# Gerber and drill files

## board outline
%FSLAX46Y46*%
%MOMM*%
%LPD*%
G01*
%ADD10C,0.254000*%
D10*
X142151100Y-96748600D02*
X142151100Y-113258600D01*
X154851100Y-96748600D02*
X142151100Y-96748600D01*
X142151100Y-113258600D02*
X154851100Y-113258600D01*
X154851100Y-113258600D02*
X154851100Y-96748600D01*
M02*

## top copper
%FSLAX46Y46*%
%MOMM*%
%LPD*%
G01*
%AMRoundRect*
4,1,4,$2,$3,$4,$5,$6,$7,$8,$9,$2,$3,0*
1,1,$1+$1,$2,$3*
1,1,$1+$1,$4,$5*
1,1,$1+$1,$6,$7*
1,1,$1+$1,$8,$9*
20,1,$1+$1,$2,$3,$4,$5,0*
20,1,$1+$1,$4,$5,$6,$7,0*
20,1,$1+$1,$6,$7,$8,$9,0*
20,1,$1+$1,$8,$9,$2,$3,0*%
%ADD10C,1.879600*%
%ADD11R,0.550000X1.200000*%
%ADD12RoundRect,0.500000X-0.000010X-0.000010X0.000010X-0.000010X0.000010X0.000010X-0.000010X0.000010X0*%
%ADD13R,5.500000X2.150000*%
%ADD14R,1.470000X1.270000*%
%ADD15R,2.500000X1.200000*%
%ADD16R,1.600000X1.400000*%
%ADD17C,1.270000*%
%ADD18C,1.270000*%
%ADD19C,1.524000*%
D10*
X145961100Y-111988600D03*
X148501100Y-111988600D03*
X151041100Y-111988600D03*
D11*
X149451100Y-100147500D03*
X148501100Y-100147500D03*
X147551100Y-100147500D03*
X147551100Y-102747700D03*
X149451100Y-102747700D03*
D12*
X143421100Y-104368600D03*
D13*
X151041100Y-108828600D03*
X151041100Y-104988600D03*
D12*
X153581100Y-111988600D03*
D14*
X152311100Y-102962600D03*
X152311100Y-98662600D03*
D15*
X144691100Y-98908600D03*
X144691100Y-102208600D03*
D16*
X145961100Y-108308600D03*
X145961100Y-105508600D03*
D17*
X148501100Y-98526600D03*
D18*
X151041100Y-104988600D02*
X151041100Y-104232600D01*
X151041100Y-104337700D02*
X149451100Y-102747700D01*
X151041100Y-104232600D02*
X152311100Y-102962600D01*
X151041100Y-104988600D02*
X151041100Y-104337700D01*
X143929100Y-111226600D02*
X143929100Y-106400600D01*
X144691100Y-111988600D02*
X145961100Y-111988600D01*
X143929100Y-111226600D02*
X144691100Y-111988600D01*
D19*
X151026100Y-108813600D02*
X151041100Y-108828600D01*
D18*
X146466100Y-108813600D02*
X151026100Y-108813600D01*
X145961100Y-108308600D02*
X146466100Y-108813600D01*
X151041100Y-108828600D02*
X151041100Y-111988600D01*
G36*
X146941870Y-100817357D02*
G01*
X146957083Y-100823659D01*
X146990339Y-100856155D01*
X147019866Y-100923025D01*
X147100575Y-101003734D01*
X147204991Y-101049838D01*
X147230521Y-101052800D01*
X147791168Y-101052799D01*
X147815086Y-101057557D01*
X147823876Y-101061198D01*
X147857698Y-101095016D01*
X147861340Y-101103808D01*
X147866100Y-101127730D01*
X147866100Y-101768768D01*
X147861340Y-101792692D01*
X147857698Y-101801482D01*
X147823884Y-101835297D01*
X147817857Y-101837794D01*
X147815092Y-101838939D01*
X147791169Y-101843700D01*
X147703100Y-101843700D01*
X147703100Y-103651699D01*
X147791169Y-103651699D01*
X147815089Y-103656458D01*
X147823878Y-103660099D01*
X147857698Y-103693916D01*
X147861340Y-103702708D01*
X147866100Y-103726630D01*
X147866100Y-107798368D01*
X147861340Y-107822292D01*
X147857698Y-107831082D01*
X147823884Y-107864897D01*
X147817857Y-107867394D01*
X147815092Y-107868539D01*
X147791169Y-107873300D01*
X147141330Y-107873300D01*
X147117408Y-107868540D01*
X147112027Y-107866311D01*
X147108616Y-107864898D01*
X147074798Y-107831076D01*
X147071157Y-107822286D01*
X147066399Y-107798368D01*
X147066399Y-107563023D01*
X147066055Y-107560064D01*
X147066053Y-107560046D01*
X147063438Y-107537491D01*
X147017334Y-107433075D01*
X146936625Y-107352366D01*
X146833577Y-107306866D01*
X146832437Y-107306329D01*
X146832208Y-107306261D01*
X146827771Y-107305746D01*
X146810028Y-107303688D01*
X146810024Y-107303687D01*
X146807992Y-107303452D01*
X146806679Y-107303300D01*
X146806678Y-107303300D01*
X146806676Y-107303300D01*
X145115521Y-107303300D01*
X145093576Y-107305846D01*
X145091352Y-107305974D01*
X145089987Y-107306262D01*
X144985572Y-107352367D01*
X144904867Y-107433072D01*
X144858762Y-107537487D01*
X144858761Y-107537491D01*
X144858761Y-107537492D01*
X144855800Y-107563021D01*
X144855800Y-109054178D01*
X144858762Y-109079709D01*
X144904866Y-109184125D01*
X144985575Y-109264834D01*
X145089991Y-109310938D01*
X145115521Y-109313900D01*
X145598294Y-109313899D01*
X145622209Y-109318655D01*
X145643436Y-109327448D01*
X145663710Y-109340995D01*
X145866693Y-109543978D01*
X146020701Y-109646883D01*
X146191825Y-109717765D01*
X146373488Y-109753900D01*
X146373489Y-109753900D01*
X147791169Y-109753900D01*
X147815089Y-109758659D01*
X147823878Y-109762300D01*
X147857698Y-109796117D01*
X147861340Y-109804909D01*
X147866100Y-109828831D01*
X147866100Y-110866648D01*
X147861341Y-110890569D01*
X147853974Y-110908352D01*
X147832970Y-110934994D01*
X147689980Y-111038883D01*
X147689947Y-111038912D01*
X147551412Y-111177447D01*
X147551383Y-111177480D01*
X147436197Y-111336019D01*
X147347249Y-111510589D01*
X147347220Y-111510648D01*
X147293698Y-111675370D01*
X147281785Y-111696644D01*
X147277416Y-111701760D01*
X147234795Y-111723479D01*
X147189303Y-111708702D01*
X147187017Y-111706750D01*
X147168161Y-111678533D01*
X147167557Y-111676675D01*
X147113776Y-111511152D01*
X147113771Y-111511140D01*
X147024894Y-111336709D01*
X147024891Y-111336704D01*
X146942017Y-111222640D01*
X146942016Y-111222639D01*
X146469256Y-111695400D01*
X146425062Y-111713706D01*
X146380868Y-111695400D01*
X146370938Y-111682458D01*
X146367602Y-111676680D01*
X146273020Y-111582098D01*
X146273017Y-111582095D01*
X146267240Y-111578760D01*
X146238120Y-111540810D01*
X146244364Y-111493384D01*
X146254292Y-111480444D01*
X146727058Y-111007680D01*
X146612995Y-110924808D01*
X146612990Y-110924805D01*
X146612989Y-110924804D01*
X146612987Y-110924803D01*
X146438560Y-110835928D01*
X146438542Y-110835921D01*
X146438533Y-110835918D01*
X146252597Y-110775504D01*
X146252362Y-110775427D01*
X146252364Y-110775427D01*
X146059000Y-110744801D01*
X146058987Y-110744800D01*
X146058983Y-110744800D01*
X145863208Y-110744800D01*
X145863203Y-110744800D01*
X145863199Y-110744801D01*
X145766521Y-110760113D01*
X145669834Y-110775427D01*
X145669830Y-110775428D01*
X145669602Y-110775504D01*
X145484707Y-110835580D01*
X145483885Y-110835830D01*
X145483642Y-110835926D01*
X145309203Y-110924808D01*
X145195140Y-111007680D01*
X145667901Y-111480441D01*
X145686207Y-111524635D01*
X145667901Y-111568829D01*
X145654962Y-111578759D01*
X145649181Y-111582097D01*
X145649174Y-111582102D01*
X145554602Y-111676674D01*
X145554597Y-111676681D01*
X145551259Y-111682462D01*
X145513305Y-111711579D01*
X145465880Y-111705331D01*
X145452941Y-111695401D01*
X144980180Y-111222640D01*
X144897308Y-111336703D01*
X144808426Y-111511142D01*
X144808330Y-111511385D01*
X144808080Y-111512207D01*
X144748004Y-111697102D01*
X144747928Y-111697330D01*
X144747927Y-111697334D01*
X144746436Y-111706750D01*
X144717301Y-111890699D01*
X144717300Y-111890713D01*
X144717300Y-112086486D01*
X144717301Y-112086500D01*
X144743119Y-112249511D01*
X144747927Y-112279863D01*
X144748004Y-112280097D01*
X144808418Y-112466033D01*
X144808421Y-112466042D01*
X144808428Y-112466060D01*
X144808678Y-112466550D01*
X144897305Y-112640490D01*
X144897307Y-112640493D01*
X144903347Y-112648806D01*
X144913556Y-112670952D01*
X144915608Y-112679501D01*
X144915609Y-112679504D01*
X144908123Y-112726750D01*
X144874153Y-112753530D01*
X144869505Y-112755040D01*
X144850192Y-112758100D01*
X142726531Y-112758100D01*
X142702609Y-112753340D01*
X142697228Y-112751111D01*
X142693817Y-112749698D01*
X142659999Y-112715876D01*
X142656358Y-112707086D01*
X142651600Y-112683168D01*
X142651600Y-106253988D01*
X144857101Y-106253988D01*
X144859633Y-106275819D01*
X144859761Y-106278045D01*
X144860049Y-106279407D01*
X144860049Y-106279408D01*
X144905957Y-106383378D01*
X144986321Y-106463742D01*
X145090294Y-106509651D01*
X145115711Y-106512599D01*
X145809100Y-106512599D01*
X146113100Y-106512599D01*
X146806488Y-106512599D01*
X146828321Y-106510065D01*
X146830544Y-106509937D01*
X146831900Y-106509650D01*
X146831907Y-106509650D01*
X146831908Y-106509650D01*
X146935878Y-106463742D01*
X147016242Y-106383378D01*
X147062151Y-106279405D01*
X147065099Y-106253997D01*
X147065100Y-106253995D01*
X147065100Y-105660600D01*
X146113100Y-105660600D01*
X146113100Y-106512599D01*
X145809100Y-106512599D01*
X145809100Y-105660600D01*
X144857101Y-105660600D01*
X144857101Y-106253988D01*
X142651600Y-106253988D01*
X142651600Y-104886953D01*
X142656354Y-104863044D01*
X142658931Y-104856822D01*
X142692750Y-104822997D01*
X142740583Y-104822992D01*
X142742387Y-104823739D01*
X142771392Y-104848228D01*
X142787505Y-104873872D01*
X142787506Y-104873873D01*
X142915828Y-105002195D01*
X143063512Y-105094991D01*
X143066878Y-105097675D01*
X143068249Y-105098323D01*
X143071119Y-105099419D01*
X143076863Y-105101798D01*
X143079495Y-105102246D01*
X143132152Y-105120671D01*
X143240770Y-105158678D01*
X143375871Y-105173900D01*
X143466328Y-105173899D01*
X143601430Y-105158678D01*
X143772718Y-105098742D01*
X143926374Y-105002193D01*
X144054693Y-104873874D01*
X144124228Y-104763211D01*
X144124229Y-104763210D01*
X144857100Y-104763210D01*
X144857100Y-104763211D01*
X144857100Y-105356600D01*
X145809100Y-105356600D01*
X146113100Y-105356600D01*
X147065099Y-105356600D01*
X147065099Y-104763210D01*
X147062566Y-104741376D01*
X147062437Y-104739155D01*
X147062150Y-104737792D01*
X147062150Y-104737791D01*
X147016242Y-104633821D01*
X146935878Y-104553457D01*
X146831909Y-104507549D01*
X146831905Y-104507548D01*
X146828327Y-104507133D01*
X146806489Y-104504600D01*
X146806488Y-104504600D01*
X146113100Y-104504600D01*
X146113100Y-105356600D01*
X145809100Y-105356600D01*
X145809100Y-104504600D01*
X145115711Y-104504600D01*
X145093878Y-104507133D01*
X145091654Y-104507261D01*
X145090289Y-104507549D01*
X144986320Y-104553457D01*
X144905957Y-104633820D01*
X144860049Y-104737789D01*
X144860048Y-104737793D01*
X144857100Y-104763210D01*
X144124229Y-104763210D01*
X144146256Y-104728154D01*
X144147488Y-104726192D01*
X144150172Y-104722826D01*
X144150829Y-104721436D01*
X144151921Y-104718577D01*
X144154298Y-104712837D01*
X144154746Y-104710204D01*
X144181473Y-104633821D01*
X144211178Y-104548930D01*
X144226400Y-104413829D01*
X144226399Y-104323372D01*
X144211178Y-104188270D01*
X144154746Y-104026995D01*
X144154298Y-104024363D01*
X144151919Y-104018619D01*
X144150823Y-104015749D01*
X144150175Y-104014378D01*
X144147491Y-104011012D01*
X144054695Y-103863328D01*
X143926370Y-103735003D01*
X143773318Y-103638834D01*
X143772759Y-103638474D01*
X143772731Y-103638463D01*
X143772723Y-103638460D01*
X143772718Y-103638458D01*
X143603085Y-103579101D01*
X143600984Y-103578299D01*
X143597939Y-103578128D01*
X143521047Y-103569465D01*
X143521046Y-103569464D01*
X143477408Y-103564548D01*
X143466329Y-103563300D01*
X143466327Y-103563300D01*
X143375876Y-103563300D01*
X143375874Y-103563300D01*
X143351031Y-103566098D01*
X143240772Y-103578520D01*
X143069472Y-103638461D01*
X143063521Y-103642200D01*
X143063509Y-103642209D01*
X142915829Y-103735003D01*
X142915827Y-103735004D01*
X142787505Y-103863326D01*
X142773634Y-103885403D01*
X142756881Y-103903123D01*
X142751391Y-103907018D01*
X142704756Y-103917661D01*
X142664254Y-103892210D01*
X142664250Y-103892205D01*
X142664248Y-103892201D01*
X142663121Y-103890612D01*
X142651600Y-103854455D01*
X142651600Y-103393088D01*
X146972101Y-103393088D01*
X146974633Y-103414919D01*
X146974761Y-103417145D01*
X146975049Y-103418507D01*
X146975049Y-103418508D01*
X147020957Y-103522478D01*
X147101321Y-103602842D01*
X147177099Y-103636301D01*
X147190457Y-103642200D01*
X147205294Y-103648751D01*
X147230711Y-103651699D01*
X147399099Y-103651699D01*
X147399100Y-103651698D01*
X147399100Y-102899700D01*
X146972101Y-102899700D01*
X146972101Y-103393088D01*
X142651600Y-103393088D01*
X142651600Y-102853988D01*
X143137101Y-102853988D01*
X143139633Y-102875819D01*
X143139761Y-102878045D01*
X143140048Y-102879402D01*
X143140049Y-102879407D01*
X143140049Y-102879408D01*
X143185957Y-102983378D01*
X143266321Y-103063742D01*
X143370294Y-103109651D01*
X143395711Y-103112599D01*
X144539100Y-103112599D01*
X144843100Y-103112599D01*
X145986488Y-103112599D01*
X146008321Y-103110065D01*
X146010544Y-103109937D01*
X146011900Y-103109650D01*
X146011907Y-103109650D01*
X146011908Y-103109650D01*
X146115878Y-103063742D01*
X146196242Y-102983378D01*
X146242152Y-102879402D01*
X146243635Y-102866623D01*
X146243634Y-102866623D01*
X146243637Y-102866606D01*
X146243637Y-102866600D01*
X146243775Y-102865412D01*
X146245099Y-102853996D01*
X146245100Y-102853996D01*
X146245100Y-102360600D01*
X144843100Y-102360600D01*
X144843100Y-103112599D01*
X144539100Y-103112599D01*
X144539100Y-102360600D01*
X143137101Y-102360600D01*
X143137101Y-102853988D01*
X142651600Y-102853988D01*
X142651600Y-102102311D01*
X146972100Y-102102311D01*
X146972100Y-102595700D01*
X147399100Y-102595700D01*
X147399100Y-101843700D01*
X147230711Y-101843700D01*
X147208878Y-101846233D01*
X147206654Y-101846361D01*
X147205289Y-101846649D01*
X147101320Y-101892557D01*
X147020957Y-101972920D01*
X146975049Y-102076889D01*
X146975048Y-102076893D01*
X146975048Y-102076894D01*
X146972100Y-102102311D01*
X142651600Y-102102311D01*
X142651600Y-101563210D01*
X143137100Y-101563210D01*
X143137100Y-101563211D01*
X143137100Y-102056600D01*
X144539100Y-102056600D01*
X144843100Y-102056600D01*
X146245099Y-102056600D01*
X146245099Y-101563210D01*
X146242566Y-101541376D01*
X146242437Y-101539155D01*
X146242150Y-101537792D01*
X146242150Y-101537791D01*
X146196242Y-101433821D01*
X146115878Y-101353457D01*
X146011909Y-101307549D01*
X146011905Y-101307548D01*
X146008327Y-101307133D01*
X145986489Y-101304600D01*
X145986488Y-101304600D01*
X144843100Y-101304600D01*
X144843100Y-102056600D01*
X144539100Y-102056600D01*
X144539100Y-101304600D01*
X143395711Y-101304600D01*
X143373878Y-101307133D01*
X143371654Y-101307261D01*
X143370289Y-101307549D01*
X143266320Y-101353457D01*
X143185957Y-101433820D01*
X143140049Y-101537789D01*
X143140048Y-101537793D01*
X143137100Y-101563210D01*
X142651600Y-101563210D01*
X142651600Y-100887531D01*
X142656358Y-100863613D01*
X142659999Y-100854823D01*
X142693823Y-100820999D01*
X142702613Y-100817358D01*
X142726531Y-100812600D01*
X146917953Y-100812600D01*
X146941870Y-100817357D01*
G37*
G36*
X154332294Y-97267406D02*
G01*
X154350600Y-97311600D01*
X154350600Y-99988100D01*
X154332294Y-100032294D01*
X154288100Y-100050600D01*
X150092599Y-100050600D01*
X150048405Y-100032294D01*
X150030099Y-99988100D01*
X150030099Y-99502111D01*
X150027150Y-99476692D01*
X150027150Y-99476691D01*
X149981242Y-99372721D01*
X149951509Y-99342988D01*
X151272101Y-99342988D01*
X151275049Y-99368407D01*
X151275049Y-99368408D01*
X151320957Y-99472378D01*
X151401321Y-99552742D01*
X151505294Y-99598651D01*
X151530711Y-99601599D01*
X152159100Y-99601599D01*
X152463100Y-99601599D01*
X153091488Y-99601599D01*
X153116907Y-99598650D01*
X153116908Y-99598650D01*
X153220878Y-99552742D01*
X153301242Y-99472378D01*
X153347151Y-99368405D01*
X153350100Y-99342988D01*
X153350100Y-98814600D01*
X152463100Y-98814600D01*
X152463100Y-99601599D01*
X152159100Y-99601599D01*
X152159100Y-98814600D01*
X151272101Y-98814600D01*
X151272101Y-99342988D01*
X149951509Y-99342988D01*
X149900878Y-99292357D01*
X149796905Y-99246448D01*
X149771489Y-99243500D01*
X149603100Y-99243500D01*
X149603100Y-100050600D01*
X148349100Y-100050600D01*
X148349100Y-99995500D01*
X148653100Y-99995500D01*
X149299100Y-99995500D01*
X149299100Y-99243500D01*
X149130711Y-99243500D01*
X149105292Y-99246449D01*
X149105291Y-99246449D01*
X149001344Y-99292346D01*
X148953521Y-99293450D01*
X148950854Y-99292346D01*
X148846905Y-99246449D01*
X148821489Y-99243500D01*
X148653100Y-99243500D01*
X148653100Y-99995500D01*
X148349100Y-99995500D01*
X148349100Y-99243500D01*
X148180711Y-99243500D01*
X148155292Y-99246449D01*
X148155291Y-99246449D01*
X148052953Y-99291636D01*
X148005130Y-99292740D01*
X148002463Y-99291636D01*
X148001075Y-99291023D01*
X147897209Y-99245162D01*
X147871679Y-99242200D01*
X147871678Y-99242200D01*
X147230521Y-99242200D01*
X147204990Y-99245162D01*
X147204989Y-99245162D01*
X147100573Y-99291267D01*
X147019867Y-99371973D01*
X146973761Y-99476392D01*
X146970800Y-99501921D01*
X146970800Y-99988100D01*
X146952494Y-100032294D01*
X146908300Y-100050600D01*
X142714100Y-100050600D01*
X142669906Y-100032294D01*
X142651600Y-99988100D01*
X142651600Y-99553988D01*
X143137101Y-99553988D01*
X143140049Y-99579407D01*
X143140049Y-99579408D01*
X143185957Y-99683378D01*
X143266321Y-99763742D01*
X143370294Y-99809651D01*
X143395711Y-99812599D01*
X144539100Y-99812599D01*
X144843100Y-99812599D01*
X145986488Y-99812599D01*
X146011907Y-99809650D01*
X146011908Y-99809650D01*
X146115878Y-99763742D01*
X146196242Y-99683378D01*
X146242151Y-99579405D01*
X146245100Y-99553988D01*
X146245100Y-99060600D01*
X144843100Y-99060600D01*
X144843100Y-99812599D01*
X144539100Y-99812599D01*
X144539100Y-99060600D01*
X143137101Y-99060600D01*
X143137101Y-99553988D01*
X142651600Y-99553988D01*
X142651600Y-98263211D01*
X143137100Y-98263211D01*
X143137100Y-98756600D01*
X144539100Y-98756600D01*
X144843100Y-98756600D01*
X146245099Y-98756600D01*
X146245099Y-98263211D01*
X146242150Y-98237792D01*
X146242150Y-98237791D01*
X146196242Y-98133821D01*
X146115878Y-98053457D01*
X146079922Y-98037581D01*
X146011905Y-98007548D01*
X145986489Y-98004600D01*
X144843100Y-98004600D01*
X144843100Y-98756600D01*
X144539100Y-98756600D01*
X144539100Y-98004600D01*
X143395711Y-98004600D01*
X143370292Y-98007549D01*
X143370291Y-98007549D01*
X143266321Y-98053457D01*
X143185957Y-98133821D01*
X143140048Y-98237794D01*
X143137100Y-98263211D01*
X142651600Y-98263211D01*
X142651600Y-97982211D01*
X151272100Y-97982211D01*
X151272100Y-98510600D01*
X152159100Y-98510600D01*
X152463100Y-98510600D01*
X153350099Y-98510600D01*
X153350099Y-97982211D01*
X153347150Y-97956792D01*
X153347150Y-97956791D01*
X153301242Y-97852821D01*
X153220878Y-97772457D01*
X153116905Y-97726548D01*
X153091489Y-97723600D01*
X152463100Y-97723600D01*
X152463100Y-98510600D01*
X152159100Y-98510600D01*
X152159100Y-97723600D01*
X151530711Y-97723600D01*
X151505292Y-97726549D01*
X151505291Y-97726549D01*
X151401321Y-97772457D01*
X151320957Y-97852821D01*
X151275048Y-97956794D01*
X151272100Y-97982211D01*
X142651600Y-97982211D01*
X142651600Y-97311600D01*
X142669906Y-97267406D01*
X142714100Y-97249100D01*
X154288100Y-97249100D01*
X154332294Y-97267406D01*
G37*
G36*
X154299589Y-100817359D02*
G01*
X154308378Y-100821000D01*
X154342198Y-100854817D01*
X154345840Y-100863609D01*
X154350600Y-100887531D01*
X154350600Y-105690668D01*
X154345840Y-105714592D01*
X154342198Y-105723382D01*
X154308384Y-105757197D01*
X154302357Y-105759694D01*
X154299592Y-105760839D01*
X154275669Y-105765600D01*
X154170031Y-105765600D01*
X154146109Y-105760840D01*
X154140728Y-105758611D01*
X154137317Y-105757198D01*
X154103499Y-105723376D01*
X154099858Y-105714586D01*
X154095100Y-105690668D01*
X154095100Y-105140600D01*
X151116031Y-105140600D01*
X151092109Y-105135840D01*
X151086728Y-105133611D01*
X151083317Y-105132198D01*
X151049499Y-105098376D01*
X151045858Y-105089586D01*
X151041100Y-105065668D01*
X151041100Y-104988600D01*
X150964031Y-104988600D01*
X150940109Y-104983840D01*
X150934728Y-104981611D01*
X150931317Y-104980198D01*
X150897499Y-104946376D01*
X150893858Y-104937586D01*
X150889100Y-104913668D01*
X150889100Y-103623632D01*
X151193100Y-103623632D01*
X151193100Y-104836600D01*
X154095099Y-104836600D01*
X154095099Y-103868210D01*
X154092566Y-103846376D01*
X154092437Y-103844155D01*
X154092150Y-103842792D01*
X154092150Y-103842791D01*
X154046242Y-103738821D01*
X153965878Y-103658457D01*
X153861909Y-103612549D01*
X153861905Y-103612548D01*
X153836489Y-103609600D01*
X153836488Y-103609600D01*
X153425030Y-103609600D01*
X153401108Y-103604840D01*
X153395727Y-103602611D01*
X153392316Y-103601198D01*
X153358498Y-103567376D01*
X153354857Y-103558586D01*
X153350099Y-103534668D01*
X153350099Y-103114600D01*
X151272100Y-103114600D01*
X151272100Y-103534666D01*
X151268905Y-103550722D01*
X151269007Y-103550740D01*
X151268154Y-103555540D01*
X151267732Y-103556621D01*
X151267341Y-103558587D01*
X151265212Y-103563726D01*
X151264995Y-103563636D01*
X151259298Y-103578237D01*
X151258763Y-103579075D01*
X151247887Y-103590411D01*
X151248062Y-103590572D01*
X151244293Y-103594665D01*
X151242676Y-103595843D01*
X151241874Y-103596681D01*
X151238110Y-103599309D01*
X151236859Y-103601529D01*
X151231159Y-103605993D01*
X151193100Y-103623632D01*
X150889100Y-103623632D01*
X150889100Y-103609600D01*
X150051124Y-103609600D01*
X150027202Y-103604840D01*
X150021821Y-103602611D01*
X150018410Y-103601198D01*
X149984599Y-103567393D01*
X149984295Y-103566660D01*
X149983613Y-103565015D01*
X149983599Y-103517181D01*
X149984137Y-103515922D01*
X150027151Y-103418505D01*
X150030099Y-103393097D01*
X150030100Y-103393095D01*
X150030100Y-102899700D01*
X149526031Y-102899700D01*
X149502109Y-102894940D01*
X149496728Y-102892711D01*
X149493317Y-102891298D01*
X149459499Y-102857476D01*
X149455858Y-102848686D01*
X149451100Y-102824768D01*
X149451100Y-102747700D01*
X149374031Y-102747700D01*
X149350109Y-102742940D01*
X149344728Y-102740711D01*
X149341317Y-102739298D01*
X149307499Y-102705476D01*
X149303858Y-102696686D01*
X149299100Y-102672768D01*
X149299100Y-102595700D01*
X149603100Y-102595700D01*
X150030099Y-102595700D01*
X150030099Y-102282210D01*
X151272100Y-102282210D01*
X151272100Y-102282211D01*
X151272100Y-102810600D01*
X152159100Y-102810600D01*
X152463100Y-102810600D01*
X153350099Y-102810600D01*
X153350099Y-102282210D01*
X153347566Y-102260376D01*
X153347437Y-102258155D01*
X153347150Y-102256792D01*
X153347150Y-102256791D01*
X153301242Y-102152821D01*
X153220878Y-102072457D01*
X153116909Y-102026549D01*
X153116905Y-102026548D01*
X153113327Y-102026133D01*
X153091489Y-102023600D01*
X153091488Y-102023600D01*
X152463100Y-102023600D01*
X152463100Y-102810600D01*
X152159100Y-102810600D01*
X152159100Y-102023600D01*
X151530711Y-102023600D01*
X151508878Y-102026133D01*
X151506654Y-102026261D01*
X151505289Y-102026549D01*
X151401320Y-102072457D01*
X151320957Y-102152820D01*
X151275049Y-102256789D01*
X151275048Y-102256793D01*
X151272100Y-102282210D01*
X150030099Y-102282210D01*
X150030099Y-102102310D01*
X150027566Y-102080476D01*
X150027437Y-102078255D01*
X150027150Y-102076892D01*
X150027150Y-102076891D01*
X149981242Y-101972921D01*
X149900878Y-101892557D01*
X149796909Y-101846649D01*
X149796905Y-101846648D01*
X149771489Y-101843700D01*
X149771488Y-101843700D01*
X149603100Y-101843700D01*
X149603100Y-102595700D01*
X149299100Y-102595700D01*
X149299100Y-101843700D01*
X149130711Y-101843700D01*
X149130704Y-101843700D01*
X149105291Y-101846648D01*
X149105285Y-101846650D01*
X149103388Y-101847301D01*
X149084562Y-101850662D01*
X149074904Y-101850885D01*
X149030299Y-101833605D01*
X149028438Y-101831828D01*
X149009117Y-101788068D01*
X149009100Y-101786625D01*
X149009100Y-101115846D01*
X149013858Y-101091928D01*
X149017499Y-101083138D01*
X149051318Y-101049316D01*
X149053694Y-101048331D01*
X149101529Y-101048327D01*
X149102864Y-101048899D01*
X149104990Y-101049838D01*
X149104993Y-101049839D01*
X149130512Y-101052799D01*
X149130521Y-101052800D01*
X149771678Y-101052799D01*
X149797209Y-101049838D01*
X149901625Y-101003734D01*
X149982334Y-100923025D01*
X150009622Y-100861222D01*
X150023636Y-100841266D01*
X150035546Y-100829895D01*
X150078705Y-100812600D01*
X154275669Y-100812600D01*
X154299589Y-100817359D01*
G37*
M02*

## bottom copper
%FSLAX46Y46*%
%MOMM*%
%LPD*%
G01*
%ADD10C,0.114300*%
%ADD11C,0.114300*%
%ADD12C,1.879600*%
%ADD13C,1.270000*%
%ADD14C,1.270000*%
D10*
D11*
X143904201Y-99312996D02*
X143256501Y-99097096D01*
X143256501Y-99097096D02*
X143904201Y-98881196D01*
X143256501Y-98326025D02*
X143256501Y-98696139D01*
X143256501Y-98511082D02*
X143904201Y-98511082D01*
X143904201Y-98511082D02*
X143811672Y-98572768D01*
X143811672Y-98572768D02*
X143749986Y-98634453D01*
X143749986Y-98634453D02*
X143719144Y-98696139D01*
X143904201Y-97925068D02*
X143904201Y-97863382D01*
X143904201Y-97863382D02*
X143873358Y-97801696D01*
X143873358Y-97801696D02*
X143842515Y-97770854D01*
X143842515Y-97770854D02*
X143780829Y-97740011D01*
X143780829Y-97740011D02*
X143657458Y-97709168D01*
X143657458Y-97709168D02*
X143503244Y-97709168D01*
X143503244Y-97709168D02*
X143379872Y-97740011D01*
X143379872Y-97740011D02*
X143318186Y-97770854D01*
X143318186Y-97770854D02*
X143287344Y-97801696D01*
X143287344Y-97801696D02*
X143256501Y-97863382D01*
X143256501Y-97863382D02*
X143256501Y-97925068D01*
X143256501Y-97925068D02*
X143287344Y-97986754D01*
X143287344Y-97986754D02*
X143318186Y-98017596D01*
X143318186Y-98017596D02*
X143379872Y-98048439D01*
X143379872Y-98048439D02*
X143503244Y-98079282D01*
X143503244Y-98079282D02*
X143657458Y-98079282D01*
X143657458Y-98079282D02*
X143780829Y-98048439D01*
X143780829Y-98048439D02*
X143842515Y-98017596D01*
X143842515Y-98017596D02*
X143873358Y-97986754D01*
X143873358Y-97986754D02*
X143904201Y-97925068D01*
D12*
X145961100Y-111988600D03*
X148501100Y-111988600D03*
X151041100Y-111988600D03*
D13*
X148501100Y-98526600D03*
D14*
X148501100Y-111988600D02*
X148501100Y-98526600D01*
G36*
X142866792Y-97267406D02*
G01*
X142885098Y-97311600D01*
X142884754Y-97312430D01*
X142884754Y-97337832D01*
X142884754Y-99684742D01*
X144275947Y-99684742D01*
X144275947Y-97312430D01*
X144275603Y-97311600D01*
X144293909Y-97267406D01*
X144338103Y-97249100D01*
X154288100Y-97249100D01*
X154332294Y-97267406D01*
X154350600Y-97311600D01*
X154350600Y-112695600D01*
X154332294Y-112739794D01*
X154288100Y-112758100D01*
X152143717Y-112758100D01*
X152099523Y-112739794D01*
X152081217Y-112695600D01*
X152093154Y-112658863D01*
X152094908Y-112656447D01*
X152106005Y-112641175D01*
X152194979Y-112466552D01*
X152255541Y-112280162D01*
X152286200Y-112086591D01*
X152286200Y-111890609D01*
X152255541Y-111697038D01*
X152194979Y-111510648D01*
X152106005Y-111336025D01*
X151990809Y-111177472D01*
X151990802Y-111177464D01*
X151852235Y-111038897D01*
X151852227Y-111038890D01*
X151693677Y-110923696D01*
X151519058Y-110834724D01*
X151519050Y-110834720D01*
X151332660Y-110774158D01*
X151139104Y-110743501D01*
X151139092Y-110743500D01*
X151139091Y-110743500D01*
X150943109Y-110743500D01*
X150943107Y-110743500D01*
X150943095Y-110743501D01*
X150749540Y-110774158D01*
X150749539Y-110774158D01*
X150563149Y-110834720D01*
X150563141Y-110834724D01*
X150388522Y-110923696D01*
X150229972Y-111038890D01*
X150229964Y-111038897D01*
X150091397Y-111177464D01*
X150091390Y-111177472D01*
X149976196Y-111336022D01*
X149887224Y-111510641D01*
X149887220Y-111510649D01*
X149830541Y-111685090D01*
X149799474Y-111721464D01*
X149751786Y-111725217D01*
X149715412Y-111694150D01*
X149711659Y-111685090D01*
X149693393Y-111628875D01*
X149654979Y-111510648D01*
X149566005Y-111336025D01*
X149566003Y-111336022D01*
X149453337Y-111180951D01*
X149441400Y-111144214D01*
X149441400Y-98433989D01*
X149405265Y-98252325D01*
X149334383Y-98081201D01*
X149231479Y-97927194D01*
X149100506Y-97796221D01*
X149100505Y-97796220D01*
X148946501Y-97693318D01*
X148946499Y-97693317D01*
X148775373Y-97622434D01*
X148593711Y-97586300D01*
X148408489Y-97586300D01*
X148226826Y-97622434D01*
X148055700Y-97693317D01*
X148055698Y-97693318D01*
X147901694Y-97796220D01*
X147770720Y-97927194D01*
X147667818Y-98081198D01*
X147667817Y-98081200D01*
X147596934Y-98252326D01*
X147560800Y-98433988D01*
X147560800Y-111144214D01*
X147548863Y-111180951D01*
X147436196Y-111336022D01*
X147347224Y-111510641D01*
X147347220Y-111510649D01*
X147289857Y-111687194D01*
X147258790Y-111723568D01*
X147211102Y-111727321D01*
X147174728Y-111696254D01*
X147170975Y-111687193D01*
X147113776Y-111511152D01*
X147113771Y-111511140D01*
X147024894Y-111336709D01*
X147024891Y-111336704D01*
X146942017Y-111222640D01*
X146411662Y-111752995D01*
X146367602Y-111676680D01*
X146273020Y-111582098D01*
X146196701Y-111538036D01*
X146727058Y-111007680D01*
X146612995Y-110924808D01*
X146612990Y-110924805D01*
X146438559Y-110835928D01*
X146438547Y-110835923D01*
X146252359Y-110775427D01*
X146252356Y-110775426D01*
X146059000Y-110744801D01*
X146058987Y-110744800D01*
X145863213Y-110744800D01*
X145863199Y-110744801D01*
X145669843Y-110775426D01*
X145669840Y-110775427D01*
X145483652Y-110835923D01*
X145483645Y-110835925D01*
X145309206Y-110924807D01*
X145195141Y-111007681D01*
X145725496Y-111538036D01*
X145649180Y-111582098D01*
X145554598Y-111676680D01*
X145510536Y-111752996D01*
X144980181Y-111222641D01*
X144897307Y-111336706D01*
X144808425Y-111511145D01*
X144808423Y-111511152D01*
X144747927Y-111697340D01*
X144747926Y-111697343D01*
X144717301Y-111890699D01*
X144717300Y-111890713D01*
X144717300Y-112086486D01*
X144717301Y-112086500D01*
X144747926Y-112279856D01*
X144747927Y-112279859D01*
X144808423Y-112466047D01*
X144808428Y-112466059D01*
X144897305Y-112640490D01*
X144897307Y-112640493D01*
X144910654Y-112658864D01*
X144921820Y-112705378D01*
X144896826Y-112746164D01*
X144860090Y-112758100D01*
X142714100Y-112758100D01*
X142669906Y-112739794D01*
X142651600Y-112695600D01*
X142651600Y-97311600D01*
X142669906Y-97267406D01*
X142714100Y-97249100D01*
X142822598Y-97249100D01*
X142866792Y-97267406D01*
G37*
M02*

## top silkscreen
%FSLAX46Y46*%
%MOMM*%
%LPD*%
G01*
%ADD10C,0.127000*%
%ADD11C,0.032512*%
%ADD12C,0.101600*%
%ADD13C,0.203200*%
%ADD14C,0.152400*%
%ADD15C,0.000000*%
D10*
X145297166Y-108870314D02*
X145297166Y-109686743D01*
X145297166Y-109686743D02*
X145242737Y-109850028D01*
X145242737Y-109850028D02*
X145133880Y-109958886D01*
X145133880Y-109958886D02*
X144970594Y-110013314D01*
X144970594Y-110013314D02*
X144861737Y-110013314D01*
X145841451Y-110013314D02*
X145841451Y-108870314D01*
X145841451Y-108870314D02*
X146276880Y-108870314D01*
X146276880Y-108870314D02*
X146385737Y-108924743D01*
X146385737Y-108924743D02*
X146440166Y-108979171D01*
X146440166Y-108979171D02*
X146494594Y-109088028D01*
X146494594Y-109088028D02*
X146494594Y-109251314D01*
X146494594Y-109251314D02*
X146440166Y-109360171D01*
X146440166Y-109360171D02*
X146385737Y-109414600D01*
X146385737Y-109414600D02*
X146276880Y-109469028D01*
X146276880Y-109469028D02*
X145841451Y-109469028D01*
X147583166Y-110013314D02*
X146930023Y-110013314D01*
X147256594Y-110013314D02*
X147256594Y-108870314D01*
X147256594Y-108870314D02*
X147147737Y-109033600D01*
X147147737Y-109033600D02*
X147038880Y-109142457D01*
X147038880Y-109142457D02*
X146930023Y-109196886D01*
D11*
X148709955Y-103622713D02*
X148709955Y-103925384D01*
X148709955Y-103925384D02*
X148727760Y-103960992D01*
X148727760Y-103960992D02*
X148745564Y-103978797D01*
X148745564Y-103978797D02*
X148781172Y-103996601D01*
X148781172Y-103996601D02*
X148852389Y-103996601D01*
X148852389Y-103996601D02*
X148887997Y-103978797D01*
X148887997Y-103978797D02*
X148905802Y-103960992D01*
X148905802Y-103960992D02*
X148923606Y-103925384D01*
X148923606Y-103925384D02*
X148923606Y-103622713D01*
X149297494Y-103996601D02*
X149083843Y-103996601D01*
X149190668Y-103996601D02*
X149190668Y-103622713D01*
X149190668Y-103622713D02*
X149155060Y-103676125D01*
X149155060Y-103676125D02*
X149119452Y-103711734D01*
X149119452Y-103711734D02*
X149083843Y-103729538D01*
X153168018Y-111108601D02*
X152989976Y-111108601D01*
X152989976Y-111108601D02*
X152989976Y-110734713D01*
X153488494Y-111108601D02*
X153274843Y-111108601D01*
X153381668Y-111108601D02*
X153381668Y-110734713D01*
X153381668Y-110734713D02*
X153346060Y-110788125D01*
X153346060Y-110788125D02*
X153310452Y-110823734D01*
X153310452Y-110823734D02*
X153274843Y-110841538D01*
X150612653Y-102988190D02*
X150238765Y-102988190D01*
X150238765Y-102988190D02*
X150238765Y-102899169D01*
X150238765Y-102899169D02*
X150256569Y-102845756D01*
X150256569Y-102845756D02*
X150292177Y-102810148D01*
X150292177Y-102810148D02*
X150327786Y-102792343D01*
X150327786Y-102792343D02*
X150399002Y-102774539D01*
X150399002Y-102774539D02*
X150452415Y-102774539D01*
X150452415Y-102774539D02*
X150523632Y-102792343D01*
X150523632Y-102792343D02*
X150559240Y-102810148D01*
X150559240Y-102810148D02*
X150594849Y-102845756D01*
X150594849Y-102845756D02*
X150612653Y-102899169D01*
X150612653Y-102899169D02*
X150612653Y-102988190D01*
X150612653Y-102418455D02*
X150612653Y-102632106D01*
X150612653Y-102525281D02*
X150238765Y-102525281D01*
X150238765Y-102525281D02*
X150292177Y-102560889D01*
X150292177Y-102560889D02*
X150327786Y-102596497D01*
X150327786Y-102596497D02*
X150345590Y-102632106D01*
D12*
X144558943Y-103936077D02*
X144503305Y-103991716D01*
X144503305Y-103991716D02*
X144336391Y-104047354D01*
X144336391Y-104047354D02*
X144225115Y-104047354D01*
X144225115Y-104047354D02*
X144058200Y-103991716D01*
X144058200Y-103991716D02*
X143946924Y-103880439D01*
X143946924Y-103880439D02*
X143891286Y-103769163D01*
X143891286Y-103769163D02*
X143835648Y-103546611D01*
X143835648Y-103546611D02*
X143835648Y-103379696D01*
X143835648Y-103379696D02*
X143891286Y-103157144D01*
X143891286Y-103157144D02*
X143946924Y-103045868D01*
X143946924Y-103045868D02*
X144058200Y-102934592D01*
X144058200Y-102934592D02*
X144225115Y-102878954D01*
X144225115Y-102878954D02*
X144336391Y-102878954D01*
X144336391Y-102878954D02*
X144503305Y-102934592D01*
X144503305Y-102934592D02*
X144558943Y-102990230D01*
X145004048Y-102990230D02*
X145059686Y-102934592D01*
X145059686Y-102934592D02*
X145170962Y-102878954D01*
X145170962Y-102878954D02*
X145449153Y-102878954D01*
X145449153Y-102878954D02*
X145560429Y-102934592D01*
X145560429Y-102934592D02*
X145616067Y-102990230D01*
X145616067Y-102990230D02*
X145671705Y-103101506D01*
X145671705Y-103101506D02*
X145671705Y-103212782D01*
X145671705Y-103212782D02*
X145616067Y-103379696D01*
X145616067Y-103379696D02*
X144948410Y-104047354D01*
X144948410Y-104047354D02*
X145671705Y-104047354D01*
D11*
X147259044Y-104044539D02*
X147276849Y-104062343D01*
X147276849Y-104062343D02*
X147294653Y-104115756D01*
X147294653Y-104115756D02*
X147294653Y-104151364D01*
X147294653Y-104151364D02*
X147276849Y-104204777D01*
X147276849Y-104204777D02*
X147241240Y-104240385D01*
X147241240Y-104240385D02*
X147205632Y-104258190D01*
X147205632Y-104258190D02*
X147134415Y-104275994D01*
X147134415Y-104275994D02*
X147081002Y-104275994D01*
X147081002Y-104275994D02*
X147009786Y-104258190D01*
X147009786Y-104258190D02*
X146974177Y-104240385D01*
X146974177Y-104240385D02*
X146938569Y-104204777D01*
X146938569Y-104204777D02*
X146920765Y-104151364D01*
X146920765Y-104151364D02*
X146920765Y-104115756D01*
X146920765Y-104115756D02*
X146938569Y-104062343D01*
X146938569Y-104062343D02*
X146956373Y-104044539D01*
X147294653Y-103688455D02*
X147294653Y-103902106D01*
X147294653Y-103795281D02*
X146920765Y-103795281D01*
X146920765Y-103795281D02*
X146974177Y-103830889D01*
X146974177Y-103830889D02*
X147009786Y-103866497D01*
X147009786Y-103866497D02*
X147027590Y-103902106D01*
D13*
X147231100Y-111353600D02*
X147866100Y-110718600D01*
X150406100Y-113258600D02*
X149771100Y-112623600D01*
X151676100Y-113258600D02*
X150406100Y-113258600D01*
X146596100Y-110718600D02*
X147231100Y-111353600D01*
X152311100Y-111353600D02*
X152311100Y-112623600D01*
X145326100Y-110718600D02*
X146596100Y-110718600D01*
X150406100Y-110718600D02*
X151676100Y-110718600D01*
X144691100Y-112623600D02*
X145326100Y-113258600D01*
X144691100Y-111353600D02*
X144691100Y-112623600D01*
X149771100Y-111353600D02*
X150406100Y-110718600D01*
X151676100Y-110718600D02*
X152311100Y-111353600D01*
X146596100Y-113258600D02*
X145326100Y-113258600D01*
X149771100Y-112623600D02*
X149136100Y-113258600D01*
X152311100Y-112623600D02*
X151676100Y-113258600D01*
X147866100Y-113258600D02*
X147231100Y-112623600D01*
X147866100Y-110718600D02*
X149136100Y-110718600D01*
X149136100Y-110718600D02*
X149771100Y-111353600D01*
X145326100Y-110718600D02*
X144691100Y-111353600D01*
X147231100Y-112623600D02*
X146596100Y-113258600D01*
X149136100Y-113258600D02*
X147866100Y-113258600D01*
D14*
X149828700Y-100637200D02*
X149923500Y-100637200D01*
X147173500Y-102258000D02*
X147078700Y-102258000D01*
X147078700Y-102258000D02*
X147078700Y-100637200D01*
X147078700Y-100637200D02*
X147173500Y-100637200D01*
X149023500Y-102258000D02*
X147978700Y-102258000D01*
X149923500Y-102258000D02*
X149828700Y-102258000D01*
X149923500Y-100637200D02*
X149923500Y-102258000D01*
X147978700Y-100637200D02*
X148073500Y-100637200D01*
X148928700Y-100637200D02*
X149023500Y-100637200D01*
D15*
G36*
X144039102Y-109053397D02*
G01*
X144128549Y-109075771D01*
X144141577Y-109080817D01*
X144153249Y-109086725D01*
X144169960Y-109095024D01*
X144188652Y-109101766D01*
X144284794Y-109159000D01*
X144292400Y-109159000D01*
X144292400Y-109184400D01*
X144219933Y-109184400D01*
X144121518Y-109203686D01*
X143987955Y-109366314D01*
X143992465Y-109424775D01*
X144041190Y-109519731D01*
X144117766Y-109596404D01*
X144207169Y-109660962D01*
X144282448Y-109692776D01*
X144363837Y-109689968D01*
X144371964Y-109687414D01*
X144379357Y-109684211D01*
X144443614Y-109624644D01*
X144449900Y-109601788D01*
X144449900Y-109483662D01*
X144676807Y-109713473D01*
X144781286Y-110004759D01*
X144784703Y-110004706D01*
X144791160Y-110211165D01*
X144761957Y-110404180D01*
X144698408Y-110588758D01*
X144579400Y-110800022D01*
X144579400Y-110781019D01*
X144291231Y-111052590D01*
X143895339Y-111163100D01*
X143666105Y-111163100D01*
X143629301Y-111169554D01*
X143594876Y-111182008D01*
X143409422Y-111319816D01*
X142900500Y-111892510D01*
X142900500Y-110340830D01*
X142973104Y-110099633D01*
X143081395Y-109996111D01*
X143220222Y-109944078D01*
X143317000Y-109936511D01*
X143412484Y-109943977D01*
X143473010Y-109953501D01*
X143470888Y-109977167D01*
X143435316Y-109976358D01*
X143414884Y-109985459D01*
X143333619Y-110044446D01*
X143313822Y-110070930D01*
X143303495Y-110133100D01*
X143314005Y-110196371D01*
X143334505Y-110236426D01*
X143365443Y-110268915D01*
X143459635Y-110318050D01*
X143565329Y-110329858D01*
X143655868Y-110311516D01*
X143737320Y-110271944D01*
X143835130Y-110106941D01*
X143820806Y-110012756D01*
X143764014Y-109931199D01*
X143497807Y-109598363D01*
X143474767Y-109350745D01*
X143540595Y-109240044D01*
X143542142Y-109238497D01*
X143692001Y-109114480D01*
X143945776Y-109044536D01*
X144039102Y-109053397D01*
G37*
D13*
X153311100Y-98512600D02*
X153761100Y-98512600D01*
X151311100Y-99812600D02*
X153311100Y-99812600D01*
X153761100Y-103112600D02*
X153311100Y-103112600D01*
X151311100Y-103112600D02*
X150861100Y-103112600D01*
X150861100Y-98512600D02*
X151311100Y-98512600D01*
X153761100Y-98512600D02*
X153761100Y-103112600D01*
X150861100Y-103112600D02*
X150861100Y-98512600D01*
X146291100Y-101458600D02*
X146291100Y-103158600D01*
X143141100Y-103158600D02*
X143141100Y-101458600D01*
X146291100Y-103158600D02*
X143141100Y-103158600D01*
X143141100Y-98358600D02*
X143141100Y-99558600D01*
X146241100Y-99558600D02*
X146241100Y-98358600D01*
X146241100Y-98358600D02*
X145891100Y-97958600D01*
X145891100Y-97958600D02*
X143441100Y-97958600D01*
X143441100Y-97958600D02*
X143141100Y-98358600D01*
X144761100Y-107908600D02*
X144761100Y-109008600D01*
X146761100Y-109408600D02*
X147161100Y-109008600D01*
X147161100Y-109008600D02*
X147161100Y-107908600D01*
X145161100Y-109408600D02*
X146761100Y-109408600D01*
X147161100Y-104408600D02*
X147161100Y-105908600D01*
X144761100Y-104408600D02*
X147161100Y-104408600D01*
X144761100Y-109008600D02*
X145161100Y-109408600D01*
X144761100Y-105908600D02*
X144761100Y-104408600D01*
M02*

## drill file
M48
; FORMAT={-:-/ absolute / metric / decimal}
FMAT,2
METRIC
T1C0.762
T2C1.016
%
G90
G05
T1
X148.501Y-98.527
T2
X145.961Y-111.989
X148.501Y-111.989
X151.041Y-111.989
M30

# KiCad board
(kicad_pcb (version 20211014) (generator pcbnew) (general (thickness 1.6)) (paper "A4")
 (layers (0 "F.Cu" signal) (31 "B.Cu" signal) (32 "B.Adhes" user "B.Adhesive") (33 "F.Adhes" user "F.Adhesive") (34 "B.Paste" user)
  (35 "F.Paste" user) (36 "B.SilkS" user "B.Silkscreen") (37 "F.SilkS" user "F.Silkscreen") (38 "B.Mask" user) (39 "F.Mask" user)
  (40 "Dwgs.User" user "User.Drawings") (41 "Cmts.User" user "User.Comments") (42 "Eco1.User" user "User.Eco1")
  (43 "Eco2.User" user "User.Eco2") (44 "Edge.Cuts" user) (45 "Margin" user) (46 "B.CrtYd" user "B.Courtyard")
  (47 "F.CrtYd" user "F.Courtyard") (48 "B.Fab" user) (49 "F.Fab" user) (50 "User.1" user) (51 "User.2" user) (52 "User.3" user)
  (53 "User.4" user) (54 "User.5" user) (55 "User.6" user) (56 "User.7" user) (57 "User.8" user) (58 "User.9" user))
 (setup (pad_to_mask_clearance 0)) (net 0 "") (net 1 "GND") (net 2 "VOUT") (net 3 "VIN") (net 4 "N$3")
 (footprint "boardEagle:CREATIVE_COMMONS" (layer "F.Cu") (at 129.4511 131.0386)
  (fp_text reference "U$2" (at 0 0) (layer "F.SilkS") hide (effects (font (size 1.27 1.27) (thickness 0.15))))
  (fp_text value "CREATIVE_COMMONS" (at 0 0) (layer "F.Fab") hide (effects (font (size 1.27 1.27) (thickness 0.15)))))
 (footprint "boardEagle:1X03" (layer "F.Cu") (at 145.9611 111.9886)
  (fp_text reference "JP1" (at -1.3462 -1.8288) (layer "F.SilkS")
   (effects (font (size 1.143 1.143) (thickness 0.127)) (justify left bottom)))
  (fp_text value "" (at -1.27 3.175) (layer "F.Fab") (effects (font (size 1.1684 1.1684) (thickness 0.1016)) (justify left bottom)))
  (fp_line (start 1.27 -0.635) (end 1.905 -1.27) (layer "F.SilkS") (width 0.2032))
  (fp_line (start 4.445 1.27) (end 3.81 0.635) (layer "F.SilkS") (width 0.2032))
  (fp_line (start 5.715 1.27) (end 4.445 1.27) (layer "F.SilkS") (width 0.2032))
  (fp_line (start 0.635 -1.27) (end 1.27 -0.635) (layer "F.SilkS") (width 0.2032))
  (fp_line (start 6.35 -0.635) (end 6.35 0.635) (layer "F.SilkS") (width 0.2032))
  (fp_line (start -0.635 -1.27) (end 0.635 -1.27) (layer "F.SilkS") (width 0.2032))
  (fp_line (start 4.445 -1.27) (end 5.715 -1.27) (layer "F.SilkS") (width 0.2032))
  (fp_line (start -1.27 0.635) (end -0.635 1.27) (layer "F.SilkS") (width 0.2032))
  (fp_line (start -1.27 -0.635) (end -1.27 0.635) (layer "F.SilkS") (width 0.2032))
  (fp_line (start 3.81 -0.635) (end 4.445 -1.27) (layer "F.SilkS") (width 0.2032))
  (fp_line (start 5.715 -1.27) (end 6.35 -0.635) (layer "F.SilkS") (width 0.2032))
  (fp_line (start 0.635 1.27) (end -0.635 1.27) (layer "F.SilkS") (width 0.2032))
  (fp_line (start 3.81 0.635) (end 3.175 1.27) (layer "F.SilkS") (width 0.2032))
  (fp_line (start 6.35 0.635) (end 5.715 1.27) (layer "F.SilkS") (width 0.2032))
  (fp_line (start 1.905 1.27) (end 1.27 0.635) (layer "F.SilkS") (width 0.2032))
  (fp_line (start 1.905 -1.27) (end 3.175 -1.27) (layer "F.SilkS") (width 0.2032))
  (fp_line (start 3.175 -1.27) (end 3.81 -0.635) (layer "F.SilkS") (width 0.2032))
  (fp_line (start -0.635 -1.27) (end -1.27 -0.635) (layer "F.SilkS") (width 0.2032))
  (fp_line (start 1.27 0.635) (end 0.635 1.27) (layer "F.SilkS") (width 0.2032))
  (fp_line (start 3.175 1.27) (end 1.905 1.27) (layer "F.SilkS") (width 0.2032))
  (pad "1" thru_hole circle (at 0 0 90) (size 1.8796 1.8796) (drill 1.016) (layers *.Cu *.Mask) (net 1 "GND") (solder_mask_margin 0.1016))
  (pad "2" thru_hole circle (at 2.54 0 90) (size 1.8796 1.8796) (drill 1.016) (layers *.Cu *.Mask) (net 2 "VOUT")
   (solder_mask_margin 0.1016))
  (pad "3" thru_hole circle (at 5.08 0 90) (size 1.8796 1.8796) (drill 1.016) (layers *.Cu *.Mask) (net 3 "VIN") (solder_mask_margin 0.1016)))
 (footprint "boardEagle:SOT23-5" (layer "F.Cu") (at 148.5011 101.4476 180)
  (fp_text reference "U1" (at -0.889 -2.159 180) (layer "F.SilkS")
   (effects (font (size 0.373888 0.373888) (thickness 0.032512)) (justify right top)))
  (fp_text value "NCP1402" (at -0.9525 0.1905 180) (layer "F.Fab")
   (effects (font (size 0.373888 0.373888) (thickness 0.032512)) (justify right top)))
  (fp_line (start -1.3276 0.8104) (end -1.4224 0.8104) (layer "F.SilkS") (width 0.1524))
  (fp_line (start 1.3276 -0.8104) (end 1.4224 -0.8104) (layer "F.SilkS") (width 0.1524))
  (fp_line (start 1.4224 -0.8104) (end 1.4224 0.8104) (layer "F.SilkS") (width 0.1524))
  (fp_line (start 1.4224 0.8104) (end 1.3276 0.8104) (layer "F.SilkS") (width 0.1524))
  (fp_line (start -0.5224 -0.8104) (end 0.5224 -0.8104) (layer "F.SilkS") (width 0.1524))
  (fp_line (start -1.4224 -0.8104) (end -1.3276 -0.8104) (layer "F.SilkS") (width 0.1524))
  (fp_line (start -1.4224 0.8104) (end -1.4224 -0.8104) (layer "F.SilkS") (width 0.1524))
  (fp_line (start 0.5224 0.8104) (end 0.4276 0.8104) (layer "F.SilkS") (width 0.1524))
  (fp_line (start -0.4276 0.8104) (end -0.5224 0.8104) (layer "F.SilkS") (width 0.1524))
  (pad "1" smd rect (at -0.95 1.3001 180) (size 0.55 1.2) (layers "F.Cu" "F.Paste" "F.Mask") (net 2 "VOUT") (solder_mask_margin 0.1016))
  (pad "2" smd rect (at 0 1.3001 180) (size 0.55 1.2) (layers "F.Cu" "F.Paste" "F.Mask") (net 2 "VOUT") (solder_mask_margin 0.1016))
  (pad "3" smd rect (at 0.95 1.3001 180) (size 0.55 1.2) (layers "F.Cu" "F.Paste" "F.Mask") (solder_mask_margin 0.1016))
  (pad "4" smd rect (at 0.95 -1.3001 180) (size 0.55 1.2) (layers "F.Cu" "F.Paste" "F.Mask") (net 1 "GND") (solder_mask_margin 0.1016))
  (pad "5" smd rect (at -0.95 -1.3001 180) (size 0.55 1.2) (layers "F.Cu" "F.Paste" "F.Mask") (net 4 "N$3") (solder_mask_margin 0.1016)))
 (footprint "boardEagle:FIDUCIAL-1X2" (layer "F.Cu") (at 143.4211 104.3686)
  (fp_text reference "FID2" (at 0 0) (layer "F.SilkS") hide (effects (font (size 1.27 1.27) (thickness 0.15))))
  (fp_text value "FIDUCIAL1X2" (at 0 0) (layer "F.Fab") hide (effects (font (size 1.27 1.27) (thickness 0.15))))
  (pad "1" smd roundrect (at 0 0) (size 1 1) (layers "F.Cu" "F.Mask") (roundrect_rratio 0.5) (solder_mask_margin 0.1016)))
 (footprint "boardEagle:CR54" (layer "F.Cu") (at 151.0411 106.9086 180)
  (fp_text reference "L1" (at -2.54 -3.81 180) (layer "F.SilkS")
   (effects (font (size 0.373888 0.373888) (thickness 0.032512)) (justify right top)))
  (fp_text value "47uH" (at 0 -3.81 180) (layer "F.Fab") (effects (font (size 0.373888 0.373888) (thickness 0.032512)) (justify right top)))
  (pad "P$1" smd rect (at 0 -1.92 180) (size 5.5 2.15) (layers "F.Cu" "F.Paste" "F.Mask") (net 3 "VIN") (solder_mask_margin 0.1016))
  (pad "P$2" smd rect (at 0 1.92 180) (size 5.5 2.15) (layers "F.Cu" "F.Paste" "F.Mask") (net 4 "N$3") (solder_mask_margin 0.1016)))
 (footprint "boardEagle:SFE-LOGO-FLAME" (layer "F.Cu") (at 142.9131 111.8616)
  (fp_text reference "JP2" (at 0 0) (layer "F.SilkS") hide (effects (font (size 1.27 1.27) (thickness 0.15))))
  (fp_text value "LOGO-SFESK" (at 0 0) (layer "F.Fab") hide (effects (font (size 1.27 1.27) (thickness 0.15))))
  (fp_poly
   (pts (xy 1.126002 -2.808203) (xy 1.215449 -2.785829) (xy 1.228477 -2.780783) (xy 1.240149 -2.774875) (xy 1.25686 -2.766576)
    (xy 1.275552 -2.759834) (xy 1.371694 -2.7026) (xy 1.3793 -2.7026) (xy 1.3793 -2.6772) (xy 1.306833 -2.6772) (xy 1.208418 -2.657914)
    (xy 1.074855 -2.495286) (xy 1.079365 -2.436825) (xy 1.12809 -2.341869) (xy 1.204666 -2.265196) (xy 1.294069 -2.200638)
    (xy 1.369348 -2.168824) (xy 1.450737 -2.171632) (xy 1.458864 -2.174186) (xy 1.466257 -2.177389) (xy 1.530514 -2.236956)
    (xy 1.5368 -2.259812) (xy 1.5368 -2.377938) (xy 1.763707 -2.148127) (xy 1.868186 -1.856841) (xy 1.871603 -1.856894)
    (xy 1.87806 -1.650435) (xy 1.848857 -1.45742) (xy 1.785308 -1.272842) (xy 1.6663 -1.061578) (xy 1.6663 -1.080581) (xy 1.378131 -0.80901)
    (xy 0.982239 -0.6985) (xy 0.753005 -0.6985) (xy 0.716201 -0.692046) (xy 0.681776 -0.679592) (xy 0.496322 -0.541784) (xy -0.0126 0.03091)
    (xy -0.0126 -1.52077) (xy 0.060004 -1.761967) (xy 0.168295 -1.865489) (xy 0.307122 -1.917522) (xy 0.4039 -1.925089)
    (xy 0.499384 -1.917623) (xy 0.55991 -1.908099) (xy 0.557788 -1.884433) (xy 0.522216 -1.885242) (xy 0.501784 -1.876141)
    (xy 0.420519 -1.817154) (xy 0.400722 -1.79067) (xy 0.390395 -1.7285) (xy 0.400905 -1.665229) (xy 0.421405 -1.625174)
    (xy 0.452343 -1.592685) (xy 0.546535 -1.54355) (xy 0.652229 -1.531742) (xy 0.742768 -1.550084) (xy 0.82422 -1.589656)
    (xy 0.92203 -1.754659) (xy 0.907706 -1.848844) (xy 0.850914 -1.930401) (xy 0.584707 -2.263237) (xy 0.561667 -2.510855)
    (xy 0.627495 -2.621556) (xy 0.629042 -2.623103) (xy 0.778901 -2.74712) (xy 1.032676 -2.817064))
   (layer "F.SilkS") (width 0) (fill solid)))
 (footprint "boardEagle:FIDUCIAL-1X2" (layer "F.Cu") (at 153.5811 111.9886)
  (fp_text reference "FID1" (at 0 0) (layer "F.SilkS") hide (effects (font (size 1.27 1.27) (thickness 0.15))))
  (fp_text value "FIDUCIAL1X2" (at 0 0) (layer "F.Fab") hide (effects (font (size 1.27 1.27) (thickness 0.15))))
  (pad "1" smd roundrect (at 0 0) (size 1 1) (layers "F.Cu" "F.Mask") (roundrect_rratio 0.5) (solder_mask_margin 0.1016)))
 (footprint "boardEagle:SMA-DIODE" (layer "F.Cu") (at 152.3111 100.8126 90)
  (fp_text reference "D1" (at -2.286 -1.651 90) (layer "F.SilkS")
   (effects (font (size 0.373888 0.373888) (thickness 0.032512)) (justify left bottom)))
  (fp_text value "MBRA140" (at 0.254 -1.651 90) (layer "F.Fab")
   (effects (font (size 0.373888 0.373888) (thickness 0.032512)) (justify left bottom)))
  (fp_line (start 2.3 1) (end 2.3 1.45) (layer "F.SilkS") (width 0.2032))
  (fp_line (start 1 -1) (end 1 1) (layer "F.SilkS") (width 0.2032))
  (fp_line (start -2.3 1.45) (end -2.3 1) (layer "F.SilkS") (width 0.2032))
  (fp_line (start -2.3 -1) (end -2.3 -1.45) (layer "F.SilkS") (width 0.2032))
  (fp_line (start 2.3 -1.45) (end 2.3 -1) (layer "F.SilkS") (width 0.2032))
  (fp_line (start 2.3 1.45) (end -2.3 1.45) (layer "F.SilkS") (width 0.2032))
  (fp_line (start -2.3 -1.45) (end 2.3 -1.45) (layer "F.SilkS") (width 0.2032))
  (pad "A" smd rect (at -2.15 0 270) (size 1.27 1.47) (layers "F.Cu" "F.Paste" "F.Mask") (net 4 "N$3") (solder_mask_margin 0.1016))
  (pad "C" smd rect (at 2.15 0 90) (size 1.27 1.47) (layers "F.Cu" "F.Paste" "F.Mask") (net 2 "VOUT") (solder_mask_margin 0.1016)))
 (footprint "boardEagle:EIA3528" (layer "F.Cu") (at 144.6911 100.5586 90)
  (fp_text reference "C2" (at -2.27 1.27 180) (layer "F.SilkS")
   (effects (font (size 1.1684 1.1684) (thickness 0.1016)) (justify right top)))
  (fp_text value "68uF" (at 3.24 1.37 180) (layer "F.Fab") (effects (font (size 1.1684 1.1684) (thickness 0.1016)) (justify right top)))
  (fp_line (start -0.9 1.6) (end -2.6 1.6) (layer "F.SilkS") (width 0.2032))
  (fp_line (start -2.6 -1.55) (end -0.9 -1.55) (layer "F.SilkS") (width 0.2032))
  (fp_line (start -2.6 1.6) (end -2.6 -1.55) (layer "F.SilkS") (width 0.2032))
  (fp_line (start 2.2 -1.55) (end 1 -1.55) (layer "F.SilkS") (width 0.2032))
  (fp_line (start 1 1.55) (end 2.2 1.55) (layer "F.SilkS") (width 0.2032))
  (fp_line (start 2.2 1.55) (end 2.6 1.2) (layer "F.SilkS") (width 0.2032))
  (fp_line (start 2.6 1.2) (end 2.6 -1.25) (layer "F.SilkS") (width 0.2032))
  (fp_line (start 2.6 -1.25) (end 2.2 -1.55) (layer "F.SilkS") (width 0.2032))
  (pad "A" smd rect (at 1.65 0 180) (size 2.5 1.2) (layers "F.Cu" "F.Paste" "F.Mask") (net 2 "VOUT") (solder_mask_margin 0.1016))
  (pad "C" smd rect (at -1.65 0 180) (size 2.5 1.2) (layers "F.Cu" "F.Paste" "F.Mask") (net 1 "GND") (solder_mask_margin 0.1016)))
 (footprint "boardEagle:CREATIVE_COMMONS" (layer "F.Cu") (at 43.871622 113.2586)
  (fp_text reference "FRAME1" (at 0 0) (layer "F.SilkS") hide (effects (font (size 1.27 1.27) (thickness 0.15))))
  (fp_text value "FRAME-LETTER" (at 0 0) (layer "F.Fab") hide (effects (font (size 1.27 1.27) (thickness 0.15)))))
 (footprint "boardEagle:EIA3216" (layer "F.Cu") (at 145.9611 106.9086 -90)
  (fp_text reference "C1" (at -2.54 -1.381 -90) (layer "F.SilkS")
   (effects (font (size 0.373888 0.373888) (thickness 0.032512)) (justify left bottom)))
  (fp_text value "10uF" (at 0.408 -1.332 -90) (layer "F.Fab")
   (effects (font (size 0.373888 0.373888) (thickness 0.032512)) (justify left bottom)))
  (fp_line (start 1 1.2) (end 2.1 1.2) (layer "F.SilkS") (width 0.2032))
  (fp_line (start 2.5 -0.8) (end 2.1 -1.2) (layer "F.SilkS") (width 0.2032))
  (fp_line (start 2.1 -1.2) (end 1 -1.2) (layer "F.SilkS") (width 0.2032))
  (fp_line (start 2.5 0.8) (end 2.5 -0.8) (layer "F.SilkS") (width 0.2032))
  (fp_line (start -2.5 -1.2) (end -1 -1.2) (layer "F.SilkS") (width 0.2032))
  (fp_line (start -2.5 1.2) (end -2.5 -1.2) (layer "F.SilkS") (width 0.2032))
  (fp_line (start 2.1 1.2) (end 2.5 0.8) (layer "F.SilkS") (width 0.2032))
  (fp_line (start -1 1.2) (end -2.5 1.2) (layer "F.SilkS") (width 0.2032))
  (pad "A" smd rect (at 1.4 0) (size 1.6 1.4) (layers "F.Cu" "F.Paste" "F.Mask") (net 3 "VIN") (solder_mask_margin 0.1016))
  (pad "C" smd rect (at -1.4 0) (size 1.6 1.4) (layers "F.Cu" "F.Paste" "F.Mask") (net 1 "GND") (solder_mask_margin 0.1016)))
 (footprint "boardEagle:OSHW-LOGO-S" (layer "B.Cu") (at 152.3111 99.2886 90)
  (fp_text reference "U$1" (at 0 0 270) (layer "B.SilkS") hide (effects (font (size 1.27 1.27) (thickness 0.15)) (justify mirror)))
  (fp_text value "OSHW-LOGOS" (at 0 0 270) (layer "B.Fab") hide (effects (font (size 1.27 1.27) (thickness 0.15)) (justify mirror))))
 (gr_line (start 142.1511 96.7486) (end 142.1511 113.2586) (layer "Edge.Cuts") (width 0.254))
 (gr_line (start 154.8511 96.7486) (end 142.1511 96.7486) (layer "Edge.Cuts") (width 0.254))
 (gr_line (start 142.1511 113.2586) (end 154.8511 113.2586) (layer "Edge.Cuts") (width 0.254))
 (gr_line (start 154.8511 113.2586) (end 154.8511 96.7486) (layer "Edge.Cuts") (width 0.254))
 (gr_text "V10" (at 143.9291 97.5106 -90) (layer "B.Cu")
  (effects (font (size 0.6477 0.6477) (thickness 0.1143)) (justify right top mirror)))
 (segment (start 151.0411 104.9886) (end 151.0411 104.2326) (width 1.27) (layer "F.Cu") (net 4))
 (segment (start 151.0411 104.3377) (end 149.4511 102.7477) (width 1.27) (layer "F.Cu") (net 4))
 (segment (start 151.0411 104.2326) (end 152.3111 102.9626) (width 1.27) (layer "F.Cu") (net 4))
 (segment (start 151.0411 104.9886) (end 151.0411 104.3377) (width 1.27) (layer "F.Cu") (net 4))
 (via (at 148.5011 98.5266) (size 1.27) (drill 0.762) (layers "F.Cu" "B.Cu") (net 2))
 (segment (start 148.5011 111.9886) (end 148.5011 98.5266) (width 1.27) (layer "B.Cu") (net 2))
 (segment (start 143.9291 111.2266) (end 143.9291 106.4006) (width 1.27) (layer "F.Cu") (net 1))
 (segment (start 144.6911 111.9886) (end 145.9611 111.9886) (width 1.27) (layer "F.Cu") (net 1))
 (segment (start 143.9291 111.2266) (end 144.6911 111.9886) (width 1.27) (layer "F.Cu") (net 1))
 (segment (start 151.0261 108.8136) (end 151.0411 108.8286) (width 1.524) (layer "F.Cu") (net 3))
 (segment (start 146.4661 108.8136) (end 151.0261 108.8136) (width 1.27) (layer "F.Cu") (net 3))
 (segment (start 145.9611 108.3086) (end 146.4661 108.8136) (width 1.27) (layer "F.Cu") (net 3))
 (segment (start 151.0411 108.8286) (end 151.0411 111.9886) (width 1.27) (layer "F.Cu") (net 3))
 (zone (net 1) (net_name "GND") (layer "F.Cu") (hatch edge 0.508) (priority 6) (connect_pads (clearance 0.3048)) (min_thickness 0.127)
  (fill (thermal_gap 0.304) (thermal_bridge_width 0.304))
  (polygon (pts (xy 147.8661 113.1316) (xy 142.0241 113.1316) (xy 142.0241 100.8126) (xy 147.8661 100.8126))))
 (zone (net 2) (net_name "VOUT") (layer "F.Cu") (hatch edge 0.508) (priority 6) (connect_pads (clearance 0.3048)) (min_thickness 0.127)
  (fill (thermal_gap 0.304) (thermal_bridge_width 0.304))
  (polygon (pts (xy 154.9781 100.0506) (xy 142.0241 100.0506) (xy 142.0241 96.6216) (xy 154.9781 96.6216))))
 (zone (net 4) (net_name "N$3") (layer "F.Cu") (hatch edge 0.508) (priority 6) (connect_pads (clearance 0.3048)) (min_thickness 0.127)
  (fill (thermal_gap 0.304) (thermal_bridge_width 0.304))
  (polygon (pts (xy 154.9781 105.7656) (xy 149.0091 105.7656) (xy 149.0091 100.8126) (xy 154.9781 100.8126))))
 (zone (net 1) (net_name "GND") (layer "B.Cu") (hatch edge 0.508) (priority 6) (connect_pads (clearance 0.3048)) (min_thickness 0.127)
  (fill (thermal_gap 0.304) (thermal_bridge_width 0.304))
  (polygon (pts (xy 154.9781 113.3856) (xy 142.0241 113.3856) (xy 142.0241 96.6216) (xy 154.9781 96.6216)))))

